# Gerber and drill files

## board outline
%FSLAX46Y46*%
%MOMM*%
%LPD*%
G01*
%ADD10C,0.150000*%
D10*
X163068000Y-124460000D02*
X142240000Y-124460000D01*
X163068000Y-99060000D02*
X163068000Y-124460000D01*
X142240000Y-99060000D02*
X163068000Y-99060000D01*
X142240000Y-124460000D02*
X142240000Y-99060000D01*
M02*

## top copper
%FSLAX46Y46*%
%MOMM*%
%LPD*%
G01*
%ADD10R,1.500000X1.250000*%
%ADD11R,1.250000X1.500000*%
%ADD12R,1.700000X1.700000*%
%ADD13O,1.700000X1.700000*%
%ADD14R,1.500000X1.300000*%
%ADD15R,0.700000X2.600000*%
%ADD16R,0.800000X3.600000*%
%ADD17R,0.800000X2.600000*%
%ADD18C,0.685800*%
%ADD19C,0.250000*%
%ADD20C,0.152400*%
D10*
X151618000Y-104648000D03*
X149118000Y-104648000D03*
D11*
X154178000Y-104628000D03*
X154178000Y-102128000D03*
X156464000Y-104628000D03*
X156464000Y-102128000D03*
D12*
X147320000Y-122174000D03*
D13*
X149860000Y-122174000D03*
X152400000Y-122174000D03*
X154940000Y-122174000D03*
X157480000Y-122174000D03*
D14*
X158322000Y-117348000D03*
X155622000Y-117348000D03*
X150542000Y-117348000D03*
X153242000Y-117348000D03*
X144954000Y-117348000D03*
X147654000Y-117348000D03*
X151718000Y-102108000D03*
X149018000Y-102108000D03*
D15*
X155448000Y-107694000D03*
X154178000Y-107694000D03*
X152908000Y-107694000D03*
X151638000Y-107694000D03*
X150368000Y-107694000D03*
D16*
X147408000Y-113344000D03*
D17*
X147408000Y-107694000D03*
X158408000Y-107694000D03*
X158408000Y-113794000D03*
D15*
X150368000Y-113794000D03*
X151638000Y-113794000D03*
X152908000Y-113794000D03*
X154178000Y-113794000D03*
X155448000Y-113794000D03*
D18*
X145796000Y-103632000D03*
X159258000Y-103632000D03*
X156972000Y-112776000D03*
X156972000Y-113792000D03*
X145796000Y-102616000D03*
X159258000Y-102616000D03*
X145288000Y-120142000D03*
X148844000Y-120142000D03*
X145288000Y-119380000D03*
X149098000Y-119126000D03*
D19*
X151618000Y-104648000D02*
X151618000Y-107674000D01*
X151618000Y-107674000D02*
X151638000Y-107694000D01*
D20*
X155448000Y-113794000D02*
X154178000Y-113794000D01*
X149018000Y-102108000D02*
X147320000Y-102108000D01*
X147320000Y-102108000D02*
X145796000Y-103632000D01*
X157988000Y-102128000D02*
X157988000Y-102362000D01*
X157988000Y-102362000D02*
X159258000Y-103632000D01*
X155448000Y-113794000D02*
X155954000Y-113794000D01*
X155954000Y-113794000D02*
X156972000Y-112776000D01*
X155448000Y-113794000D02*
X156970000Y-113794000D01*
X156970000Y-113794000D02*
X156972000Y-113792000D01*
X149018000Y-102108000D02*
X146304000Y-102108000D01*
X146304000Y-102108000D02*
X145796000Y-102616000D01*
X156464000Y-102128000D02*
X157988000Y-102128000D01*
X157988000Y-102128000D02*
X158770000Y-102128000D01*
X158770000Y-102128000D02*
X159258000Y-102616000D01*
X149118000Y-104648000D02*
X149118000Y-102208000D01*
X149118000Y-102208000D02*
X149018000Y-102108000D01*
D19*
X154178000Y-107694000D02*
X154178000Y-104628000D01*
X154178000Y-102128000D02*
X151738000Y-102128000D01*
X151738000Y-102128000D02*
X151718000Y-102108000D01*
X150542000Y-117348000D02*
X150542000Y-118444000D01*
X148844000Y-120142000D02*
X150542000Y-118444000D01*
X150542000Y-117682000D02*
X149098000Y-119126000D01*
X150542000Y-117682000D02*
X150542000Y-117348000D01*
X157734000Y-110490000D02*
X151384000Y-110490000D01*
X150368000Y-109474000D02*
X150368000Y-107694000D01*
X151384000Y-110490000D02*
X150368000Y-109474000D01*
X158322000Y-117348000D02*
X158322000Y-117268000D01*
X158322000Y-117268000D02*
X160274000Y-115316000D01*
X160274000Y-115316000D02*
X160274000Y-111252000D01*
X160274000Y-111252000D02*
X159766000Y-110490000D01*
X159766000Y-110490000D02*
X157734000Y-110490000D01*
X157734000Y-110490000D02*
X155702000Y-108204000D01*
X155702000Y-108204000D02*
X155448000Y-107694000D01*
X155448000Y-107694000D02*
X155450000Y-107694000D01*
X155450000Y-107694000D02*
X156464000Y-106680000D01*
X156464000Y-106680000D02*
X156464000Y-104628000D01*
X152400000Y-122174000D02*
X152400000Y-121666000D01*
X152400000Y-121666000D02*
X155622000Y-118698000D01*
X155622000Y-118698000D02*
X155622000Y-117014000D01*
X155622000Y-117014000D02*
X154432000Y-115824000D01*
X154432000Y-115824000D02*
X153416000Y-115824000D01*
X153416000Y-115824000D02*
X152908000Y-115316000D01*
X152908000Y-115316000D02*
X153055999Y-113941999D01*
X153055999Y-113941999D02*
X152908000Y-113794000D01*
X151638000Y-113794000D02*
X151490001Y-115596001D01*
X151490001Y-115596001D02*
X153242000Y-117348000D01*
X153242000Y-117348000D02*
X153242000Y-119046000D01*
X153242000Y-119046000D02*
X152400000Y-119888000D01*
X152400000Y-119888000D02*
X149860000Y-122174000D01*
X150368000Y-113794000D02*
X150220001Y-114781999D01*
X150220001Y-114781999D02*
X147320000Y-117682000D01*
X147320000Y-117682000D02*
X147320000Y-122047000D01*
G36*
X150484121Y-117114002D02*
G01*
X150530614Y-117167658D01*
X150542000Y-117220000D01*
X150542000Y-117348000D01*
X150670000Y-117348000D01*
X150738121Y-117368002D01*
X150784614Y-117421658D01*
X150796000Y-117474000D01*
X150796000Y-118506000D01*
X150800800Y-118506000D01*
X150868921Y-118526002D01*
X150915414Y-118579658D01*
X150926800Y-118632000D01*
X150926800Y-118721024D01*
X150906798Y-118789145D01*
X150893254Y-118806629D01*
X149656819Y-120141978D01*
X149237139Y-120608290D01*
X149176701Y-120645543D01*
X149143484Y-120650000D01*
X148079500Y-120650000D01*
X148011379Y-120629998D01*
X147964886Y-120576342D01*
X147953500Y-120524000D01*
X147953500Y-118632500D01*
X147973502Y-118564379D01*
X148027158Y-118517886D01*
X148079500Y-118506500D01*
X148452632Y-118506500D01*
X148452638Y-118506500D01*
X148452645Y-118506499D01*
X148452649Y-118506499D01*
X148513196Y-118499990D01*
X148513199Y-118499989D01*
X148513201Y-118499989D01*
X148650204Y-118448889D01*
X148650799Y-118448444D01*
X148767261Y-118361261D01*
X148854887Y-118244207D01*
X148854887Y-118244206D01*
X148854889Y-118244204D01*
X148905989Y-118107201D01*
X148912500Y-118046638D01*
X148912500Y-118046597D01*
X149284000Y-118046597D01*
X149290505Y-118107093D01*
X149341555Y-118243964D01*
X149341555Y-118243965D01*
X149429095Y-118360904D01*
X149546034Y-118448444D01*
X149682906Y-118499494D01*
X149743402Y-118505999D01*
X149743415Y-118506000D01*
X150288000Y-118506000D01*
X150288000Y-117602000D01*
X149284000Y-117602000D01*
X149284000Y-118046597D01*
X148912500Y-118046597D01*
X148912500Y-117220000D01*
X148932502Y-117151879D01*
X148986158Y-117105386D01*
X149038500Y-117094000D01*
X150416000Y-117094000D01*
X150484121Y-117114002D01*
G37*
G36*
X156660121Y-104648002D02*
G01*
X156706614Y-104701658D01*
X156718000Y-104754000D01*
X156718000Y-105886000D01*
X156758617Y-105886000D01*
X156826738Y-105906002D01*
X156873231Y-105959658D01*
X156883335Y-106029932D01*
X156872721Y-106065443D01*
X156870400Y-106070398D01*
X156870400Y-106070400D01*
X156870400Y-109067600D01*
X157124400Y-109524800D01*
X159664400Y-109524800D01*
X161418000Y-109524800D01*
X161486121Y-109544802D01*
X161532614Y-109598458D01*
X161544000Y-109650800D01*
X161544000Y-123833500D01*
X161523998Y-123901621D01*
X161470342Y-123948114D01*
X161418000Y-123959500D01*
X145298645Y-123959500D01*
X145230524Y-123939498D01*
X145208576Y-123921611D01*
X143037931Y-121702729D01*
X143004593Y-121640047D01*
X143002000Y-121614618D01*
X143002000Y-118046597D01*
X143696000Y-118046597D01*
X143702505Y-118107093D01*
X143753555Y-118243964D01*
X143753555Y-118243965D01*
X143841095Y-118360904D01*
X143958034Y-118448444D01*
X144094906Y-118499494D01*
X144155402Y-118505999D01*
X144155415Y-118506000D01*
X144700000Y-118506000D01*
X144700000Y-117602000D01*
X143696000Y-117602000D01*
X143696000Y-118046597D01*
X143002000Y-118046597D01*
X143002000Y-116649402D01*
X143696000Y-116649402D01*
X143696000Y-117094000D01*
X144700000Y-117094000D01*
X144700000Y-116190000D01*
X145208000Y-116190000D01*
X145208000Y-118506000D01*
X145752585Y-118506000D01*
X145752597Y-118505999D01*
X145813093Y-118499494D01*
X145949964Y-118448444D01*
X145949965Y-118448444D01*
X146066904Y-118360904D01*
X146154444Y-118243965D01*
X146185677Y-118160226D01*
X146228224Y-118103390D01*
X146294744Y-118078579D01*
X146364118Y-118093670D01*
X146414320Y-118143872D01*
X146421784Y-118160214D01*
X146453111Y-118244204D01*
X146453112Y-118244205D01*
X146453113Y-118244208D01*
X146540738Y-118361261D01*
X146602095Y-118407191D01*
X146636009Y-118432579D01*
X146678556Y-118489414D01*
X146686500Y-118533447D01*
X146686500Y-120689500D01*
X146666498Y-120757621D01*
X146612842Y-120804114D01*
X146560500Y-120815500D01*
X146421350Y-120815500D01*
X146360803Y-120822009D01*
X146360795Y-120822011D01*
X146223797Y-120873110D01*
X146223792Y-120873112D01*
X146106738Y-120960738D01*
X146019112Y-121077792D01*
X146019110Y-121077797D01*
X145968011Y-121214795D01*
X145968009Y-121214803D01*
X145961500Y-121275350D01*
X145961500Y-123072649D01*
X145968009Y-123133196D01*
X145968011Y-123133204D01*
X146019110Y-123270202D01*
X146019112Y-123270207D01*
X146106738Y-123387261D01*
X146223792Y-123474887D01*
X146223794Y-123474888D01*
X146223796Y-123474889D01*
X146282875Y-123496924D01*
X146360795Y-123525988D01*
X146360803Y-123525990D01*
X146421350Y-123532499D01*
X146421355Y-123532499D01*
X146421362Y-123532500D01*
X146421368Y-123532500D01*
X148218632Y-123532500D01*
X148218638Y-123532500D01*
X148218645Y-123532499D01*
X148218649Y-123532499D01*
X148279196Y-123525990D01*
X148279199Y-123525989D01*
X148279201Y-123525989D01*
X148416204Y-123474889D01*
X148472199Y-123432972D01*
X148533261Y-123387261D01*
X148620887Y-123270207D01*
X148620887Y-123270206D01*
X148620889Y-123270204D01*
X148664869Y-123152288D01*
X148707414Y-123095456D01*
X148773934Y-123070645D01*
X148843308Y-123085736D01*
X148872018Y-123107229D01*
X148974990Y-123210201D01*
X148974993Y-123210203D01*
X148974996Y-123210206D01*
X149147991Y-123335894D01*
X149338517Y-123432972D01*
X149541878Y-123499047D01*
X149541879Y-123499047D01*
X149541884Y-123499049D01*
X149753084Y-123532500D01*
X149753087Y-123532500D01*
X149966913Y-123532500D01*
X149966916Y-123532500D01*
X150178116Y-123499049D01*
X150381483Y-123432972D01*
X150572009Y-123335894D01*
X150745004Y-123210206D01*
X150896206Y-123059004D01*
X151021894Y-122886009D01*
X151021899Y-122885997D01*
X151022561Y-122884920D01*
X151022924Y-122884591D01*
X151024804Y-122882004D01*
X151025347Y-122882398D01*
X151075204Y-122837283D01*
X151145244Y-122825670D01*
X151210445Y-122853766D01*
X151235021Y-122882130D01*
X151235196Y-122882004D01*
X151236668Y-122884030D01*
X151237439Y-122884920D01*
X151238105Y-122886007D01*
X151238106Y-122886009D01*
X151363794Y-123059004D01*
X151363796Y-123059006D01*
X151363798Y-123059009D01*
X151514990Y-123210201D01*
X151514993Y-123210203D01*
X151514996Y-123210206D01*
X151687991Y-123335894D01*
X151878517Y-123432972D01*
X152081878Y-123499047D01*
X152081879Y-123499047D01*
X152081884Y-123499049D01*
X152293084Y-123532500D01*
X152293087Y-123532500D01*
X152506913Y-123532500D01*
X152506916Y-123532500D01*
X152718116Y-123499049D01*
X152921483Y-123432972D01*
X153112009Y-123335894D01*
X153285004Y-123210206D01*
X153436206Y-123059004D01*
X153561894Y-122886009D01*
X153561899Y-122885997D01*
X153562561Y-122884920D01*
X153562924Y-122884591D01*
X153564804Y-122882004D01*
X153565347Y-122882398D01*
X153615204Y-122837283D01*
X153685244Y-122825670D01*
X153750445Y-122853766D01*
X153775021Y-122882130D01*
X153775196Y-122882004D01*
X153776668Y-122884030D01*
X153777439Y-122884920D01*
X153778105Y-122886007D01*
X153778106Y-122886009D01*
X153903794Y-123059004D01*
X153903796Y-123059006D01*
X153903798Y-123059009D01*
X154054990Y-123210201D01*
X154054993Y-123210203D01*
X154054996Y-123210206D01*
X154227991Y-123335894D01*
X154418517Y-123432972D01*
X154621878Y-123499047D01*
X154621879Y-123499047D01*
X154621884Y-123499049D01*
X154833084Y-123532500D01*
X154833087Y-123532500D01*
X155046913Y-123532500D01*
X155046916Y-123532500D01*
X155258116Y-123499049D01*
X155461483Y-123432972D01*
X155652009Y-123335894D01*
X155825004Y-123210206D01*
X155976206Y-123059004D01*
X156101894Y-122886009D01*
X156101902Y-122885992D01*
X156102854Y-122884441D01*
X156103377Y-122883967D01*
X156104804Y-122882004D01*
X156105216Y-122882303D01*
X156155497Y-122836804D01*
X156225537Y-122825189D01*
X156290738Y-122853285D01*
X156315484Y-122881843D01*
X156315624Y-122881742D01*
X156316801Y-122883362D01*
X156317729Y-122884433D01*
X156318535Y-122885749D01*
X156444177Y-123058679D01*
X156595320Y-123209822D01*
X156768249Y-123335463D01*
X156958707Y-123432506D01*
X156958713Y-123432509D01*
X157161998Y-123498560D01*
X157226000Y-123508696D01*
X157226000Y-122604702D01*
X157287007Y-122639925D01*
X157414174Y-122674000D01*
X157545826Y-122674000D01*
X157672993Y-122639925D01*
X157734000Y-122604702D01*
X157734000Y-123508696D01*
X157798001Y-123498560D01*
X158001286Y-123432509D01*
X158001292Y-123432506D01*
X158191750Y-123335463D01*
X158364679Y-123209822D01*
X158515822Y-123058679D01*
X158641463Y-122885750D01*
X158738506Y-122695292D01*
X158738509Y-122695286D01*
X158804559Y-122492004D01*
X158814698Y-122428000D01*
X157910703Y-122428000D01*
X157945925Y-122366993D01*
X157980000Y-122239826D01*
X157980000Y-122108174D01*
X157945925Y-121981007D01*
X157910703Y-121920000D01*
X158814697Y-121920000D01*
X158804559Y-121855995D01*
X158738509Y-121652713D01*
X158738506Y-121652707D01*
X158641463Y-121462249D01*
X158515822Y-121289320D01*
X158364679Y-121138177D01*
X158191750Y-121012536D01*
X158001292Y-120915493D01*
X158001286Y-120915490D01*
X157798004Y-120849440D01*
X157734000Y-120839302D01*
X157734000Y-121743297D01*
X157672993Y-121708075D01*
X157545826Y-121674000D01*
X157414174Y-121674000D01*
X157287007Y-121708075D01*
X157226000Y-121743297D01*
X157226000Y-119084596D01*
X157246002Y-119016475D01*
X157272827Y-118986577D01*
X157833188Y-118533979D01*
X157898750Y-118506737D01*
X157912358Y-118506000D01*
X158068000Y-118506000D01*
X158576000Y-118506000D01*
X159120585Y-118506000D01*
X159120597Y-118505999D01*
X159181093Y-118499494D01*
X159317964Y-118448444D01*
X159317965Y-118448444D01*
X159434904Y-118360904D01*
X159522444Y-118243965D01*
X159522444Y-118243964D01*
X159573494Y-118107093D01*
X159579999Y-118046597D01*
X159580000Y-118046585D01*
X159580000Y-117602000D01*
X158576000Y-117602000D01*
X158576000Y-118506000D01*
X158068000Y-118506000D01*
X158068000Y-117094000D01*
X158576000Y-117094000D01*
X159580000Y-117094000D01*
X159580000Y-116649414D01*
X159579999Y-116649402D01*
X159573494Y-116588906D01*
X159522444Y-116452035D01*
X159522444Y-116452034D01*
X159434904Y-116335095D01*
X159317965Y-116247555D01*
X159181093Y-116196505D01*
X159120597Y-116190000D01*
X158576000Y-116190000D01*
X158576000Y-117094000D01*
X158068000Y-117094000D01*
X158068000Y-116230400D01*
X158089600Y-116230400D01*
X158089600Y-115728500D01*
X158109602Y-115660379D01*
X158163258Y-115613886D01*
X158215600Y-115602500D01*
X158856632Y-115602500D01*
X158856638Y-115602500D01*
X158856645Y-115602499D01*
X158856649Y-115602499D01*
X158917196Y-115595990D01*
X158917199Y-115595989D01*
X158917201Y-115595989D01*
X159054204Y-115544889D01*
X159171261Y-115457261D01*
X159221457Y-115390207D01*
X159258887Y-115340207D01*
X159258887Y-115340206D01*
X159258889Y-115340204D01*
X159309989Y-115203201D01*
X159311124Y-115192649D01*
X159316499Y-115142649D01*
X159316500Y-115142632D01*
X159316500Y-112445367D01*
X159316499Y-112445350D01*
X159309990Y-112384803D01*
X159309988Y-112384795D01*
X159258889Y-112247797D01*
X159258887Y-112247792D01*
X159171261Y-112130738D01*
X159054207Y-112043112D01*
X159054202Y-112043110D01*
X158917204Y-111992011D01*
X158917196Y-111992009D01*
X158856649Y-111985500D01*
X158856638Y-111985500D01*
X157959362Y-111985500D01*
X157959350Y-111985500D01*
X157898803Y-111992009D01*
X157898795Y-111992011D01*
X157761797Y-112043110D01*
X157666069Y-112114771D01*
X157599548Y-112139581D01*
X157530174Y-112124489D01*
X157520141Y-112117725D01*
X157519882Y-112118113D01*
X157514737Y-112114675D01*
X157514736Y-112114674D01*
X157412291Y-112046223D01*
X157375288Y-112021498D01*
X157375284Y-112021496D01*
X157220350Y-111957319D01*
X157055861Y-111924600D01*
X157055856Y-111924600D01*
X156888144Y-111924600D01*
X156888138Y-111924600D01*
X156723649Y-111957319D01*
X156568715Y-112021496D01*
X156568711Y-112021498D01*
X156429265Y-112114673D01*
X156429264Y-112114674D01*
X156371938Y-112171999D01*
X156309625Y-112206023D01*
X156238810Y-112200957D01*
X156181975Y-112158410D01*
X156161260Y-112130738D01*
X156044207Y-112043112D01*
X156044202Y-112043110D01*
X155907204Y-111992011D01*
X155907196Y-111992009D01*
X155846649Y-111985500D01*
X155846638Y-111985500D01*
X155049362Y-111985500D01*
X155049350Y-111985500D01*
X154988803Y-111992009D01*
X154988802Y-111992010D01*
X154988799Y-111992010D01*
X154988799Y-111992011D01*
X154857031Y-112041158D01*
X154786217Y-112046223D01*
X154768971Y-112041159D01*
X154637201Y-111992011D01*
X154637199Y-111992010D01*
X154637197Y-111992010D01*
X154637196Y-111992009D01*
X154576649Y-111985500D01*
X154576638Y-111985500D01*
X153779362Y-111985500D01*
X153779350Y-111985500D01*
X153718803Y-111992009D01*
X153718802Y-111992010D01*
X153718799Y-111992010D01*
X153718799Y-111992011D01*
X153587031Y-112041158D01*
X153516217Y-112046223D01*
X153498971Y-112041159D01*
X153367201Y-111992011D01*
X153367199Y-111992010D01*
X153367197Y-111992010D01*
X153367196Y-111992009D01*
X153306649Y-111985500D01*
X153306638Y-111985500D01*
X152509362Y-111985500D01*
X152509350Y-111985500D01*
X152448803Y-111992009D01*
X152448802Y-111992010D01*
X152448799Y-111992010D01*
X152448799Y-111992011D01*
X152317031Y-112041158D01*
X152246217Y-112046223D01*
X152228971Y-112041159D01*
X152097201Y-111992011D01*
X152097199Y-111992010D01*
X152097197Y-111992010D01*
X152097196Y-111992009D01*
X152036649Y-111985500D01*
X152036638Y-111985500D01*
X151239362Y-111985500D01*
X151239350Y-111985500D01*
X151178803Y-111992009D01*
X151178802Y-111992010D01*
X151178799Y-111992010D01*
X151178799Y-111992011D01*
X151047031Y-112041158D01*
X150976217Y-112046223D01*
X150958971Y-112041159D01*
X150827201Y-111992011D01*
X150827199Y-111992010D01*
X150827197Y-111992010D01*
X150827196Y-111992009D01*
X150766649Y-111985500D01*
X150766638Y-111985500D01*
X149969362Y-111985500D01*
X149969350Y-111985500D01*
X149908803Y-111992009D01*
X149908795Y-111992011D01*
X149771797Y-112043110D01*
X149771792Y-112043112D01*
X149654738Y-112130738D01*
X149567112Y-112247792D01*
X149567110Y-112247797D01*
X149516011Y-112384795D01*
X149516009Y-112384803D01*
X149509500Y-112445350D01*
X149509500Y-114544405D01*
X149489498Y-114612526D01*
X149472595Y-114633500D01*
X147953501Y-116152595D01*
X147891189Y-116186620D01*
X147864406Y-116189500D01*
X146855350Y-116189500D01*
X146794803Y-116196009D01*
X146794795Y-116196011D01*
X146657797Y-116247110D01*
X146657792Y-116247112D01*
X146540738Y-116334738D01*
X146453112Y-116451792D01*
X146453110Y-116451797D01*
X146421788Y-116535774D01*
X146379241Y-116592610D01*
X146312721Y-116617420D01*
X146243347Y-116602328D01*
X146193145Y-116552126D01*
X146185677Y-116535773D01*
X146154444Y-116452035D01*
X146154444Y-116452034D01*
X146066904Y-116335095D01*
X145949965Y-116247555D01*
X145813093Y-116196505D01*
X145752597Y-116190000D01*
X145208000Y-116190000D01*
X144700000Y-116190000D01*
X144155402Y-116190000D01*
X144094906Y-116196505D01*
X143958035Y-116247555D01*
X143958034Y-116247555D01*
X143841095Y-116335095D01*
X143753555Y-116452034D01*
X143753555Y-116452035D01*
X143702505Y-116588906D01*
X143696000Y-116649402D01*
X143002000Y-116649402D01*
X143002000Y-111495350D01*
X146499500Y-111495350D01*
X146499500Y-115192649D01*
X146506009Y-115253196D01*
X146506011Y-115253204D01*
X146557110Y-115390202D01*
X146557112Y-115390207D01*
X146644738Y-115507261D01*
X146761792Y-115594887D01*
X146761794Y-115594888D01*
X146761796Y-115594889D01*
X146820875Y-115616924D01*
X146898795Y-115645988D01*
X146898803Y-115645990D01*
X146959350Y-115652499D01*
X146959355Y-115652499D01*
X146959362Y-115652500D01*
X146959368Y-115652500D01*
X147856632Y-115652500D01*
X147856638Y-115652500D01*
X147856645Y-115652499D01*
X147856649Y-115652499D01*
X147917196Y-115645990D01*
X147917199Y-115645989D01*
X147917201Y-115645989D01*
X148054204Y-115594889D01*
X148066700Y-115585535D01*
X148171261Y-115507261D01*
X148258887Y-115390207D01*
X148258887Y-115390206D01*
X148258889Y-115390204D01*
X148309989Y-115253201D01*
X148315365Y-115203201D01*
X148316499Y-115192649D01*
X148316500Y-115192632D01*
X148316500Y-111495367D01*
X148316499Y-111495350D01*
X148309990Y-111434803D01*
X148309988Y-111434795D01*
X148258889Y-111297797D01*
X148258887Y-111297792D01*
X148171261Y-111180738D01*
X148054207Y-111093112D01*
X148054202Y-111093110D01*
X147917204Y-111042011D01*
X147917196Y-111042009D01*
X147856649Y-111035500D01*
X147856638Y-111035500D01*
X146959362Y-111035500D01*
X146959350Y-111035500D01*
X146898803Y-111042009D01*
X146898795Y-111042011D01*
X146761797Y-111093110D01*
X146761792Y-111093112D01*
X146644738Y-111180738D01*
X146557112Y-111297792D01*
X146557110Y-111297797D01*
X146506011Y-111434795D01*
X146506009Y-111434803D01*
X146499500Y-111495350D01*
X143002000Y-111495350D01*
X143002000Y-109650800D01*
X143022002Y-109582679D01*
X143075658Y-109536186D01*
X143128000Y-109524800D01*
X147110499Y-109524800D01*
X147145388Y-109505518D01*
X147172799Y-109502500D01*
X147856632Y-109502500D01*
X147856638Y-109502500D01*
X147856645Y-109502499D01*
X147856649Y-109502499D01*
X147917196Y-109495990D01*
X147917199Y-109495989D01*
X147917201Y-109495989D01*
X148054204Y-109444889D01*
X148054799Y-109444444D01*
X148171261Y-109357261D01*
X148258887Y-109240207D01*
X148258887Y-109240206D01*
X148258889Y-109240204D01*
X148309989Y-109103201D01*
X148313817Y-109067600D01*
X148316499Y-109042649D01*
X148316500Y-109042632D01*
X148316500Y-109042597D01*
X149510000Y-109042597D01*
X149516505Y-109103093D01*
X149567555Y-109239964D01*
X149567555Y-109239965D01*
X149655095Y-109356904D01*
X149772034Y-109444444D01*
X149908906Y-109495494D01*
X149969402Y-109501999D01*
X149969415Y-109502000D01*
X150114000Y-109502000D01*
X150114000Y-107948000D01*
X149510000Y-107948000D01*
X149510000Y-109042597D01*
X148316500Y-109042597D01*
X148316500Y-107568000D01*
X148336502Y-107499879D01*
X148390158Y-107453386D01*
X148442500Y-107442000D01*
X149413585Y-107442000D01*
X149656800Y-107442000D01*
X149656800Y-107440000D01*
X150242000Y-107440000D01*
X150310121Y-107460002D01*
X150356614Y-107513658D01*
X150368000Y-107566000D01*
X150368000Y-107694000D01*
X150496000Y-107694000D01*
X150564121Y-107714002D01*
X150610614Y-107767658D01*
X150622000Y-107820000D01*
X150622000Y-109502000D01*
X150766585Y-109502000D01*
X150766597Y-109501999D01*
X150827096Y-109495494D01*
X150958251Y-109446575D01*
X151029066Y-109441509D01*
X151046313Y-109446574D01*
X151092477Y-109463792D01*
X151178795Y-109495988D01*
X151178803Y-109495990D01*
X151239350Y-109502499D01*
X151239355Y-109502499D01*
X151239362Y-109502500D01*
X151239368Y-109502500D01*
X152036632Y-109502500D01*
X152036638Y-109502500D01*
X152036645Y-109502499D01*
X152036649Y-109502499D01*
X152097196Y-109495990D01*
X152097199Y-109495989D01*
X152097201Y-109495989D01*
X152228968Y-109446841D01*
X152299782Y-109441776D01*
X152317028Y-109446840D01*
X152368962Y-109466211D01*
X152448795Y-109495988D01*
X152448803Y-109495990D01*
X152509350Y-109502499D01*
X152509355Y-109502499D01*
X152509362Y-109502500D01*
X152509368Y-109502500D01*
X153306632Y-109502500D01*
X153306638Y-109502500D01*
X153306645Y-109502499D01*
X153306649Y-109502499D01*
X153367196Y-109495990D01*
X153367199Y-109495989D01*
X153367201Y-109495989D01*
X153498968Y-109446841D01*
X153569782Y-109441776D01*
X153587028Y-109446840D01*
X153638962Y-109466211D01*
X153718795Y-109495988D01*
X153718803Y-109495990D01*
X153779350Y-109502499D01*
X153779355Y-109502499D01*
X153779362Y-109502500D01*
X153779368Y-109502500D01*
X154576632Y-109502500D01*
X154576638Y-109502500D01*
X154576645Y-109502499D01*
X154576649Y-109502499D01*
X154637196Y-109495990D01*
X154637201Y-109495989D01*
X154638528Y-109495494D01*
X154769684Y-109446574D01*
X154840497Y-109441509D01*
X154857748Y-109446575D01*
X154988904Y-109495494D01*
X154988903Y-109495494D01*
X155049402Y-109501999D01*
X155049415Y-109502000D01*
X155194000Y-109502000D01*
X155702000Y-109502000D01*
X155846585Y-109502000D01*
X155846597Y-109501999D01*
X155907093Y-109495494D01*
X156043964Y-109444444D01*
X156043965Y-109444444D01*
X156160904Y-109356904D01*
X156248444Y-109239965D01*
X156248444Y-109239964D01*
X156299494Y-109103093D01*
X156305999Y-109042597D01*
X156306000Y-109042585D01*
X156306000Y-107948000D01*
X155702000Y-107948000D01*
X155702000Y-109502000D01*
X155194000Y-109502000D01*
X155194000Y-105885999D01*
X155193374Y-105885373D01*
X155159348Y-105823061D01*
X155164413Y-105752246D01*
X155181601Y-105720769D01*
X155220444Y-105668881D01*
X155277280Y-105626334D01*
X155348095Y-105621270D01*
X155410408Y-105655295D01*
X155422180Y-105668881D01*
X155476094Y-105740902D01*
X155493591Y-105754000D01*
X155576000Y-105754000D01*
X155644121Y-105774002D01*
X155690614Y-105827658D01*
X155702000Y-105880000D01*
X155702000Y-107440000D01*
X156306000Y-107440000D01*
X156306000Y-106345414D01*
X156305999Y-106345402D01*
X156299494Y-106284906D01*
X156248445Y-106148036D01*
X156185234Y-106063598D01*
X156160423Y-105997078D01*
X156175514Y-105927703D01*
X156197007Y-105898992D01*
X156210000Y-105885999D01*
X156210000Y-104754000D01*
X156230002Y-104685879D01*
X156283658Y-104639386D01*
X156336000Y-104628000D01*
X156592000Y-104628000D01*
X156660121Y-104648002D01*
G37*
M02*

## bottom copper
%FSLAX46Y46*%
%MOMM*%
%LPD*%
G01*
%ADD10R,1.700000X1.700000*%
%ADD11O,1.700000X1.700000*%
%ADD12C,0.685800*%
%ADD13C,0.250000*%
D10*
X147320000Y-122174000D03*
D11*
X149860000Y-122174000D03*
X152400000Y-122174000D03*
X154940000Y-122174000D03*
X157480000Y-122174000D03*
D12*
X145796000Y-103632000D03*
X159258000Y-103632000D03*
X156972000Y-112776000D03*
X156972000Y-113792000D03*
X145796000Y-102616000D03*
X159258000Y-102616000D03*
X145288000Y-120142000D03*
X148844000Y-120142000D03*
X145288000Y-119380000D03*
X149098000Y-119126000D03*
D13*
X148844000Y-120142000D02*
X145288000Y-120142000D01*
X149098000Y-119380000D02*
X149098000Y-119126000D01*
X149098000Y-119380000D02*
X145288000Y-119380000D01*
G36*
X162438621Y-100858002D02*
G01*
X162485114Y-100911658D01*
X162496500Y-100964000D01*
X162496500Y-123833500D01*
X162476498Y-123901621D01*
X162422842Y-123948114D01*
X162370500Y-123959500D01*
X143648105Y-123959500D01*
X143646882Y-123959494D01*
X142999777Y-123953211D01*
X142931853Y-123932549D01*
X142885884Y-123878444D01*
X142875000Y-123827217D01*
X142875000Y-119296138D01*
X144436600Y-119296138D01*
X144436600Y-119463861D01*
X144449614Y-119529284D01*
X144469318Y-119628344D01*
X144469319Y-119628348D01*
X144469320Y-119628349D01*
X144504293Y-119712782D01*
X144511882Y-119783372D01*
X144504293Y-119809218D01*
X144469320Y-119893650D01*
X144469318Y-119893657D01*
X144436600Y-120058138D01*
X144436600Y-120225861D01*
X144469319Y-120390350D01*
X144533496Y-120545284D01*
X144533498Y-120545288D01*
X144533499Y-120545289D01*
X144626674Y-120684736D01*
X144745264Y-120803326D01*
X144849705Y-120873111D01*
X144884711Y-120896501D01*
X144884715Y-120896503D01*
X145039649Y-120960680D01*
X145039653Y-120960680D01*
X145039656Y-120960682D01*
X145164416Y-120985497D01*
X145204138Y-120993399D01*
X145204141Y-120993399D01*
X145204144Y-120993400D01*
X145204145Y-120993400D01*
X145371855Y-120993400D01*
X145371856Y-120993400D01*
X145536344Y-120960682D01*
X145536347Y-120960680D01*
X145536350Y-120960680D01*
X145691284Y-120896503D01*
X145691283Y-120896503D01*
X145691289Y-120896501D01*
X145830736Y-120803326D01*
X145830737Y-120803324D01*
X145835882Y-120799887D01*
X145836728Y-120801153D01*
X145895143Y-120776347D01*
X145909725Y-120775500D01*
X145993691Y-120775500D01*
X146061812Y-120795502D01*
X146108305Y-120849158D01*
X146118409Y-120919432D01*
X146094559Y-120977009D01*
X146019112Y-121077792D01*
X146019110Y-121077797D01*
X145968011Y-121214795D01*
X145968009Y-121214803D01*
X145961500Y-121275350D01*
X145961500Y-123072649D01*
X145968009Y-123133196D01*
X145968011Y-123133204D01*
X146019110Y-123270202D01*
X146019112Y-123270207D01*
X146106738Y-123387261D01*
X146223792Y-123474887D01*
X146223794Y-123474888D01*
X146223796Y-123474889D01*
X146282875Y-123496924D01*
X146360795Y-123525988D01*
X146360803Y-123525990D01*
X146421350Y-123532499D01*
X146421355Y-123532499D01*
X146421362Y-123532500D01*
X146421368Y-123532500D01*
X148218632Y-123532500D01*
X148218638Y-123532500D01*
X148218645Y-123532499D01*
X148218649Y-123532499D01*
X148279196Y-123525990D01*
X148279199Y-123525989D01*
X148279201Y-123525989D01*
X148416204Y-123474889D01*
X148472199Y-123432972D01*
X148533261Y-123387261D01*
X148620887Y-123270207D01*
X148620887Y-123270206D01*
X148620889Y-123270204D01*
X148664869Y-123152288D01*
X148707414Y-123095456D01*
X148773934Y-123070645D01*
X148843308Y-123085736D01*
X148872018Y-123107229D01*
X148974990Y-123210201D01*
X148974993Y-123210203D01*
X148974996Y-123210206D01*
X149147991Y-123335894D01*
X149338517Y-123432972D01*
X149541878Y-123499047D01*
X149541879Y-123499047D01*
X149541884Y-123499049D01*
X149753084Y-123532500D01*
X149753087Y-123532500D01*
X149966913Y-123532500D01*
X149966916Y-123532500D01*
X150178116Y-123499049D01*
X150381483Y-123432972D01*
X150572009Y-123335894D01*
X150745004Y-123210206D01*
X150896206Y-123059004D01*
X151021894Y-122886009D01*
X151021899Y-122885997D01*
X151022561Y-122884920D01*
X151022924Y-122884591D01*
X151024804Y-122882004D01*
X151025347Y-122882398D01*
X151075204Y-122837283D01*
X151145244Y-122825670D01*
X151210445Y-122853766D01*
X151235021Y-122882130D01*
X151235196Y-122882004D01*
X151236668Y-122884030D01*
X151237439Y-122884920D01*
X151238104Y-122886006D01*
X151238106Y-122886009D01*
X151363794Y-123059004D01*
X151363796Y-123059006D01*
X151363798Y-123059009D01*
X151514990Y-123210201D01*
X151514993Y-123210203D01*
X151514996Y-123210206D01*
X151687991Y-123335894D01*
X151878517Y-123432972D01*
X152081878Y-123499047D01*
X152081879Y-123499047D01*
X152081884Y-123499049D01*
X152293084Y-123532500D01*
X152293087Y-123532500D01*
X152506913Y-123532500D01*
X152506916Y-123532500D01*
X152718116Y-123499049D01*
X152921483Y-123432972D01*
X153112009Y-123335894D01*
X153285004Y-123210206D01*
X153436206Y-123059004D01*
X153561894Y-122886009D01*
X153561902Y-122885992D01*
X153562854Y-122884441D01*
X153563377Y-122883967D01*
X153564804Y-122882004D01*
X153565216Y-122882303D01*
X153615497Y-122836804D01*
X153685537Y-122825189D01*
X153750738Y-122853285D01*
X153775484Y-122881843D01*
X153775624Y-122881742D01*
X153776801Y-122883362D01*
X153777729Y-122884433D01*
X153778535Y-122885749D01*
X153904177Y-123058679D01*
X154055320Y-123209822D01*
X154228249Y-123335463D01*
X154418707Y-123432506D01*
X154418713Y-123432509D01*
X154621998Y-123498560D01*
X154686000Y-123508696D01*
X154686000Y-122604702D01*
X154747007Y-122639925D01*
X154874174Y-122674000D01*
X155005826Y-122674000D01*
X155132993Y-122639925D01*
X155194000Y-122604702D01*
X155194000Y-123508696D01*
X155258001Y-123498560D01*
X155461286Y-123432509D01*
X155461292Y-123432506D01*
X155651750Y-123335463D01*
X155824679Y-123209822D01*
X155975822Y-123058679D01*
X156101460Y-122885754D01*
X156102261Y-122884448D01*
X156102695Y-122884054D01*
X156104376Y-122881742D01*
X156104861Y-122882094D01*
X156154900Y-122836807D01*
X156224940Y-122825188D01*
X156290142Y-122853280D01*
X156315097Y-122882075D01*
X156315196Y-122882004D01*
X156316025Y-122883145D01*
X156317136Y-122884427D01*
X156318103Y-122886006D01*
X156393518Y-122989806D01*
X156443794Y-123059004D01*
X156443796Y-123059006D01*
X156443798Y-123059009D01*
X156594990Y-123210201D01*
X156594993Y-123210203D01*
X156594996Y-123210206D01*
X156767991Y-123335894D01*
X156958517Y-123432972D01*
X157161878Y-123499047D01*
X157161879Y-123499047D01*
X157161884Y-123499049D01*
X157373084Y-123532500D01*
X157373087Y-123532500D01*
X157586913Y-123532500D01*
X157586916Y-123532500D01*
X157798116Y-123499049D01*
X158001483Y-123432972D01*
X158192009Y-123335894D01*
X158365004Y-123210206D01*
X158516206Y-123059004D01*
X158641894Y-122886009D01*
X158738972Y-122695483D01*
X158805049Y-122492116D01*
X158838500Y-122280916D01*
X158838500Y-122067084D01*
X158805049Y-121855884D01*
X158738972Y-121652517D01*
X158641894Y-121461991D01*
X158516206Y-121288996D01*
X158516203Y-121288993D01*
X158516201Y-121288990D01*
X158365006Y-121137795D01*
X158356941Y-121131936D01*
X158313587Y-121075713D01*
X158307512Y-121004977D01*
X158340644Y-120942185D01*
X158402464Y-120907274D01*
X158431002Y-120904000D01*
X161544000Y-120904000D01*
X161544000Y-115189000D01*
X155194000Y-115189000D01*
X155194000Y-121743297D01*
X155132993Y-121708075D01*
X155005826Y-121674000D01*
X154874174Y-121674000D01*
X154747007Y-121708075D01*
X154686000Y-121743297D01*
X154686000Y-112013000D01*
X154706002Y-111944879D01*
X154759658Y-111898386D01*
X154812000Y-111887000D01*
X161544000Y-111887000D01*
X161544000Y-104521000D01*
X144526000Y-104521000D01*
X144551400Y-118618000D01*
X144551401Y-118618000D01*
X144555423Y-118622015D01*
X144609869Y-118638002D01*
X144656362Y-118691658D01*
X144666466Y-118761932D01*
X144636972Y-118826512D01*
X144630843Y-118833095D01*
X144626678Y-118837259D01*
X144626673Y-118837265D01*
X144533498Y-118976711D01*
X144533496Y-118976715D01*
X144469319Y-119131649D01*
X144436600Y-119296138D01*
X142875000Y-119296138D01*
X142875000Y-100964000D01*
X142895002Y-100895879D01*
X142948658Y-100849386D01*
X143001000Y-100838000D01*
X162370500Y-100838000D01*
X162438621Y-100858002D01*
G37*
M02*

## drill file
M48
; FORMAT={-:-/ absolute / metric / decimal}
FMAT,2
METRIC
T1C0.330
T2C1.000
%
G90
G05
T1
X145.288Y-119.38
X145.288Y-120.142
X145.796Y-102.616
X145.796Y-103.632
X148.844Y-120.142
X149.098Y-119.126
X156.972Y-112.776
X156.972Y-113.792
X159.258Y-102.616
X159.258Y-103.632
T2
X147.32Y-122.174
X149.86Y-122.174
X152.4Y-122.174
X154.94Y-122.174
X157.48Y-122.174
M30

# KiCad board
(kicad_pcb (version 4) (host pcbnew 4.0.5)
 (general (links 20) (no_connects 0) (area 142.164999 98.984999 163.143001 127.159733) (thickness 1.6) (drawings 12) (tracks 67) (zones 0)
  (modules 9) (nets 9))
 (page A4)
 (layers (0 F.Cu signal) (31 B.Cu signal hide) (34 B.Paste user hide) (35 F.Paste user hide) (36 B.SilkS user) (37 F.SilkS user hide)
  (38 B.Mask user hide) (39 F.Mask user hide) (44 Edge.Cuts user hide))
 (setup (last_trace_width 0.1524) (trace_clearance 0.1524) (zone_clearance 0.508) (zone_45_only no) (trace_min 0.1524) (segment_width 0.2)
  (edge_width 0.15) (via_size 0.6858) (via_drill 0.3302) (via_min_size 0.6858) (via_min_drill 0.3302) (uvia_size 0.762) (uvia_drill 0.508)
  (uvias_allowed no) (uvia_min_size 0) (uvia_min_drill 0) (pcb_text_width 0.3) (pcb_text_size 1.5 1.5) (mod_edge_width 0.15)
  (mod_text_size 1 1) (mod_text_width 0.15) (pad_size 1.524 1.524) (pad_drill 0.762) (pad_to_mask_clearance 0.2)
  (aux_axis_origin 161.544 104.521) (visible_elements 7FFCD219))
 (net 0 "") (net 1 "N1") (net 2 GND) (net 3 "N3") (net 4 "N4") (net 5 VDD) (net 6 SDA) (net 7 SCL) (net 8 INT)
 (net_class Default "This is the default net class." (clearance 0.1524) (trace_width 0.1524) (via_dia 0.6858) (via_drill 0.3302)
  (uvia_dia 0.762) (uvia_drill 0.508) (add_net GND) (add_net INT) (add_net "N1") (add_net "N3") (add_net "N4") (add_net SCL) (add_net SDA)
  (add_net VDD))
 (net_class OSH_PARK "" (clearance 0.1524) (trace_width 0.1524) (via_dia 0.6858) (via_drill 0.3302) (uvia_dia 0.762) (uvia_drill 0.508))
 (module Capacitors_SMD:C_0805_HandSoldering (layer F.Cu) (at 150.368 104.648 180)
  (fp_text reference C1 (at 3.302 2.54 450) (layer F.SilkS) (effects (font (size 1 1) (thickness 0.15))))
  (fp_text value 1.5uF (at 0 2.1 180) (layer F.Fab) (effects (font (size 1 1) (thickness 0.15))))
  (pad 1 smd rect (at -1.25 0 180) (size 1.5 1.25) (layers F.Cu F.Paste F.Mask) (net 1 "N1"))
  (pad 2 smd rect (at 1.25 0 180) (size 1.5 1.25) (layers F.Cu F.Paste F.Mask) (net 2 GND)))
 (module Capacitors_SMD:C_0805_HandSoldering (layer F.Cu) (at 154.178 103.378 90)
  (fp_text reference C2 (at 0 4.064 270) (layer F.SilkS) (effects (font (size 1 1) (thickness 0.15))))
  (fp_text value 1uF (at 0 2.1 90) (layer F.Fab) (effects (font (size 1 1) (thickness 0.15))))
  (pad 1 smd rect (at -1.25 0 90) (size 1.5 1.25) (layers F.Cu F.Paste F.Mask) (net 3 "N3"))
  (pad 2 smd rect (at 1.25 0 90) (size 1.5 1.25) (layers F.Cu F.Paste F.Mask) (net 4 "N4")))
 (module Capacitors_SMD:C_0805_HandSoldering (layer F.Cu) (at 156.464 103.378 90)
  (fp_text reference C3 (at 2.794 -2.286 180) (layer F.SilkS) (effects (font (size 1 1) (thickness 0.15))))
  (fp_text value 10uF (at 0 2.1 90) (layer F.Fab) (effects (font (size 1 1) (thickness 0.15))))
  (pad 1 smd rect (at -1.25 0 90) (size 1.5 1.25) (layers F.Cu F.Paste F.Mask) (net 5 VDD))
  (pad 2 smd rect (at 1.25 0 90) (size 1.5 1.25) (layers F.Cu F.Paste F.Mask) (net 2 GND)))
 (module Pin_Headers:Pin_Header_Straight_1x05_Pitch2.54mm (layer F.Cu) (at 147.32 122.174 90)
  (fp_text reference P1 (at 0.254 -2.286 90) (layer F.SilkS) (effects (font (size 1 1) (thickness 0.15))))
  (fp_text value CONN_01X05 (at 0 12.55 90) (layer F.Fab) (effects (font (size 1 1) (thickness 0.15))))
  (pad 1 thru_hole rect (at 0 0 90) (size 1.7 1.7) (drill 1) (layers *.Cu *.Mask) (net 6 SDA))
  (pad 2 thru_hole oval (at 0 2.54 90) (size 1.7 1.7) (drill 1) (layers *.Cu *.Mask) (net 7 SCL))
  (pad 3 thru_hole oval (at 0 5.08 90) (size 1.7 1.7) (drill 1) (layers *.Cu *.Mask) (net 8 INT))
  (pad 4 thru_hole oval (at 0 7.62 90) (size 1.7 1.7) (drill 1) (layers *.Cu *.Mask) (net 2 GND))
  (pad 5 thru_hole oval (at 0 10.16 90) (size 1.7 1.7) (drill 1) (layers *.Cu *.Mask) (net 5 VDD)))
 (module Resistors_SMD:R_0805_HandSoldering (layer F.Cu) (at 156.972 117.348 180)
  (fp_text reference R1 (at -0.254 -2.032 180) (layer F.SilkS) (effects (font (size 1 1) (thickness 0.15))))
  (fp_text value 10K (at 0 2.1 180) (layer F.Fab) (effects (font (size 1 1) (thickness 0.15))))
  (pad 1 smd rect (at -1.35 0 180) (size 1.5 1.3) (layers F.Cu F.Paste F.Mask) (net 5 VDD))
  (pad 2 smd rect (at 1.35 0 180) (size 1.5 1.3) (layers F.Cu F.Paste F.Mask) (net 8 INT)))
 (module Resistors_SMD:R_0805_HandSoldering (layer F.Cu) (at 151.892 117.348)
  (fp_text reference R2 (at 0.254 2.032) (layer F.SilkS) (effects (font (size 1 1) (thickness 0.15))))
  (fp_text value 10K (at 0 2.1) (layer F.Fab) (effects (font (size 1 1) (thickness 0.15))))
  (pad 1 smd rect (at -1.35 0) (size 1.5 1.3) (layers F.Cu F.Paste F.Mask) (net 5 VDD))
  (pad 2 smd rect (at 1.35 0) (size 1.5 1.3) (layers F.Cu F.Paste F.Mask) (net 7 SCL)))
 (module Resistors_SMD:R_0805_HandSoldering (layer F.Cu) (at 146.304 117.348)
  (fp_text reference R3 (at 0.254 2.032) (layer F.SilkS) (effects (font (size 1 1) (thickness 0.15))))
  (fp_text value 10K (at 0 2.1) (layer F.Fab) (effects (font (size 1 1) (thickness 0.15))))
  (pad 1 smd rect (at -1.35 0) (size 1.5 1.3) (layers F.Cu F.Paste F.Mask) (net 5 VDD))
  (pad 2 smd rect (at 1.35 0) (size 1.5 1.3) (layers F.Cu F.Paste F.Mask) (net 6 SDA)))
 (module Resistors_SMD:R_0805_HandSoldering (layer F.Cu) (at 150.368 102.108 180)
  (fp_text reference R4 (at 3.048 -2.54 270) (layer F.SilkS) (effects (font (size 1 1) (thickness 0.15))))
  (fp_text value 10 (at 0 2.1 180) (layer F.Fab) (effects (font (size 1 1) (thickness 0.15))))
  (pad 1 smd rect (at -1.35 0 180) (size 1.5 1.3) (layers F.Cu F.Paste F.Mask) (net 4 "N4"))
  (pad 2 smd rect (at 1.35 0 180) (size 1.5 1.3) (layers F.Cu F.Paste F.Mask) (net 2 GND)))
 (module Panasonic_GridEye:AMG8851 (layer F.Cu) (at 152.908 110.744)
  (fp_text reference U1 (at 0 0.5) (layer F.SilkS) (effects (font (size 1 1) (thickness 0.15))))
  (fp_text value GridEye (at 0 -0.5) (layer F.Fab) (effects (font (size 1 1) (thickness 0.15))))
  (pad 9 smd rect (at 2.54 -3.05) (size 0.7 2.6) (layers F.Cu F.Paste F.Mask) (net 5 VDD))
  (pad 10 smd rect (at 1.27 -3.05) (size 0.7 2.6) (layers F.Cu F.Paste F.Mask) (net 3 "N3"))
  (pad 11 smd rect (at 0 -3.05) (size 0.7 2.6) (layers F.Cu F.Paste F.Mask))
  (pad 12 smd rect (at -1.27 -3.05) (size 0.7 2.6) (layers F.Cu F.Paste F.Mask) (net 1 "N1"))
  (pad 13 smd rect (at -2.54 -3.05) (size 0.7 2.6) (layers F.Cu F.Paste F.Mask) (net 5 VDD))
  (pad 1 smd rect (at -5.5 2.6) (size 0.8 3.6) (layers F.Cu F.Paste F.Mask))
  (pad 14 smd rect (at -5.5 -3.05) (size 0.8 2.6) (layers F.Cu F.Paste F.Mask))
  (pad 8 smd rect (at 5.5 -3.05) (size 0.8 2.6) (layers F.Cu F.Paste F.Mask))
  (pad 7 smd rect (at 5.5 3.05) (size 0.8 2.6) (layers F.Cu F.Paste F.Mask))
  (pad 2 smd rect (at -2.54 3.05) (size 0.7 2.6) (layers F.Cu F.Paste F.Mask) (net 6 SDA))
  (pad 3 smd rect (at -1.27 3.05) (size 0.7 2.6) (layers F.Cu F.Paste F.Mask) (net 7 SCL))
  (pad 4 smd rect (at 0 3.05) (size 0.7 2.6) (layers F.Cu F.Paste F.Mask) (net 8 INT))
  (pad 5 smd rect (at 1.27 3.05) (size 0.7 2.6) (layers F.Cu F.Paste F.Mask) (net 2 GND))
  (pad 6 smd rect (at 2.54 3.05) (size 0.7 2.6) (layers F.Cu F.Paste F.Mask) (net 2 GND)))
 (gr_line (start 163.068 124.46) (end 142.24 124.46) (angle 90) (layer Edge.Cuts) (width 0.15))
 (gr_line (start 163.068 99.06) (end 163.068 124.46) (angle 90) (layer Edge.Cuts) (width 0.15))
 (gr_line (start 142.24 99.06) (end 163.068 99.06) (angle 90) (layer Edge.Cuts) (width 0.15))
 (gr_line (start 142.24 124.46) (end 142.24 99.06) (angle 90) (layer Edge.Cuts) (width 0.15))
 (segment (start 151.618 104.648) (end 151.618 107.674) (width 0.25) (layer F.Cu) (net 1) (status 20))
 (segment (start 151.618 107.674) (end 151.638 107.694) (width 0.25) (layer F.Cu) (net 1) (status 30))
 (segment (start 155.448 113.794) (end 154.178 113.794) (width 0.1524) (layer F.Cu) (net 2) (status 30))
 (via (at 145.796 103.632) (size 0.6858) (drill 0.3302) (layers F.Cu B.Cu) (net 2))
 (segment (start 149.018 102.108) (end 147.32 102.108) (width 0.1524) (layer F.Cu) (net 2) (status 10))
 (segment (start 147.32 102.108) (end 145.796 103.632) (width 0.1524) (layer F.Cu) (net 2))
 (via (at 159.258 103.632) (size 0.6858) (drill 0.3302) (layers F.Cu B.Cu) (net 2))
 (segment (start 157.988 102.128) (end 157.988 102.362) (width 0.1524) (layer F.Cu) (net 2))
 (segment (start 157.988 102.362) (end 159.258 103.632) (width 0.1524) (layer F.Cu) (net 2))
 (via (at 156.972 112.776) (size 0.6858) (drill 0.3302) (layers F.Cu B.Cu) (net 2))
 (segment (start 155.448 113.794) (end 155.954 113.794) (width 0.1524) (layer F.Cu) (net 2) (status 10))
 (segment (start 155.954 113.794) (end 156.972 112.776) (width 0.1524) (layer F.Cu) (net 2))
 (via (at 156.972 113.792) (size 0.6858) (drill 0.3302) (layers F.Cu B.Cu) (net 2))
 (segment (start 155.448 113.794) (end 156.97 113.794) (width 0.1524) (layer F.Cu) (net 2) (status 10))
 (segment (start 156.97 113.794) (end 156.972 113.792) (width 0.1524) (layer F.Cu) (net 2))
 (via (at 145.796 102.616) (size 0.6858) (drill 0.3302) (layers F.Cu B.Cu) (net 2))
 (segment (start 149.018 102.108) (end 146.304 102.108) (width 0.1524) (layer F.Cu) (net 2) (status 10))
 (segment (start 146.304 102.108) (end 145.796 102.616) (width 0.1524) (layer F.Cu) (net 2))
 (via (at 159.258 102.616) (size 0.6858) (drill 0.3302) (layers F.Cu B.Cu) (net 2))
 (segment (start 156.464 102.128) (end 157.988 102.128) (width 0.1524) (layer F.Cu) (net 2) (status 10))
 (segment (start 157.988 102.128) (end 158.77 102.128) (width 0.1524) (layer F.Cu) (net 2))
 (segment (start 158.77 102.128) (end 159.258 102.616) (width 0.1524) (layer F.Cu) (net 2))
 (segment (start 149.118 104.648) (end 149.118 102.208) (width 0.1524) (layer F.Cu) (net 2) (status 30))
 (segment (start 149.118 102.208) (end 149.018 102.108) (width 0.1524) (layer F.Cu) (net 2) (status 30))
 (segment (start 154.178 107.694) (end 154.178 104.628) (width 0.25) (layer F.Cu) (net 3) (status 10))
 (segment (start 154.178 102.128) (end 151.738 102.128) (width 0.25) (layer F.Cu) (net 4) (status 30))
 (segment (start 151.738 102.128) (end 151.718 102.108) (width 0.25) (layer F.Cu) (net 4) (status 30))
 (via (at 145.288 120.142) (size 0.6858) (drill 0.3302) (layers F.Cu B.Cu) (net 5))
 (segment (start 150.542 117.348) (end 150.542 118.444) (width 0.25) (layer F.Cu) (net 5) (status 10))
 (segment (start 148.844 120.142) (end 150.542 118.444) (width 0.25) (layer F.Cu) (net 5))
 (via (at 148.844 120.142) (size 0.6858) (drill 0.3302) (layers F.Cu B.Cu) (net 5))
 (segment (start 148.844 120.142) (end 145.288 120.142) (width 0.25) (layer B.Cu) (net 5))
 (via (at 145.288 119.38) (size 0.6858) (drill 0.3302) (layers F.Cu B.Cu) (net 5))
 (segment (start 150.542 117.682) (end 149.098 119.126) (width 0.25) (layer F.Cu) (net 5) (status 10))
 (via (at 149.098 119.126) (size 0.6858) (drill 0.3302) (layers F.Cu B.Cu) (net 5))
 (segment (start 149.098 119.38) (end 149.098 119.126) (width 0.25) (layer B.Cu) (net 5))
 (segment (start 149.098 119.38) (end 145.288 119.38) (width 0.25) (layer B.Cu) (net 5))
 (segment (start 150.542 117.682) (end 150.542 117.348) (width 0.25) (layer F.Cu) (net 5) (status 30))
 (segment (start 157.734 110.49) (end 151.384 110.49) (width 0.25) (layer F.Cu) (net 5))
 (segment (start 150.368 109.474) (end 150.368 107.694) (width 0.25) (layer F.Cu) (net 5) (status 20))
 (segment (start 151.384 110.49) (end 150.368 109.474) (width 0.25) (layer F.Cu) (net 5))
 (segment (start 158.322 117.348) (end 158.322 117.268) (width 0.25) (layer F.Cu) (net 5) (status 30))
 (segment (start 158.322 117.268) (end 160.274 115.316) (width 0.25) (layer F.Cu) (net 5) (status 10))
 (segment (start 160.274 115.316) (end 160.274 111.252) (width 0.25) (layer F.Cu) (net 5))
 (segment (start 160.274 111.252) (end 159.766 110.49) (width 0.25) (layer F.Cu) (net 5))
 (segment (start 159.766 110.49) (end 157.734 110.49) (width 0.25) (layer F.Cu) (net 5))
 (segment (start 157.734 110.49) (end 155.702 108.204) (width 0.25) (layer F.Cu) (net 5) (status 20))
 (segment (start 155.702 108.204) (end 155.448 107.694) (width 0.25) (layer F.Cu) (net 5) (status 30))
 (segment (start 155.448 107.694) (end 155.45 107.694) (width 0.25) (layer F.Cu) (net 5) (status 30))
 (segment (start 155.45 107.694) (end 156.464 106.68) (width 0.25) (layer F.Cu) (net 5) (status 10))
 (segment (start 156.464 106.68) (end 156.464 104.628) (width 0.25) (layer F.Cu) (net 5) (status 20))
 (segment (start 152.4 122.174) (end 152.4 121.666) (width 0.25) (layer F.Cu) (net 8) (status 30))
 (segment (start 152.4 121.666) (end 155.622 118.698) (width 0.25) (layer F.Cu) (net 8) (status 10))
 (segment (start 155.622 118.698) (end 155.622 117.014) (width 0.25) (layer F.Cu) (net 8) (status 20))
 (segment (start 155.622 117.014) (end 154.432 115.824) (width 0.25) (layer F.Cu) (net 8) (status 10))
 (segment (start 154.432 115.824) (end 153.416 115.824) (width 0.25) (layer F.Cu) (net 8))
 (segment (start 153.416 115.824) (end 152.908 115.316) (width 0.25) (layer F.Cu) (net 8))
 (segment (start 152.908 115.316) (end 153.055999 113.941999) (width 0.25) (layer F.Cu) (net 8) (status 20))
 (segment (start 153.055999 113.941999) (end 152.908 113.794) (width 0.25) (layer F.Cu) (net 8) (status 30))
 (segment (start 151.638 113.794) (end 151.490001 115.596001) (width 0.25) (layer F.Cu) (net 7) (status 10))
 (segment (start 151.490001 115.596001) (end 153.242 117.348) (width 0.25) (layer F.Cu) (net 7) (status 20))
 (segment (start 153.242 117.348) (end 153.242 119.046) (width 0.25) (layer F.Cu) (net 7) (status 10))
 (segment (start 153.242 119.046) (end 152.4 119.888) (width 0.25) (layer F.Cu) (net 7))
 (segment (start 152.4 119.888) (end 149.86 122.174) (width 0.25) (layer F.Cu) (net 7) (status 20))
 (segment (start 150.368 113.794) (end 150.220001 114.781999) (width 0.25) (layer F.Cu) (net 6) (status 30))
 (segment (start 150.220001 114.781999) (end 147.32 117.682) (width 0.25) (layer F.Cu) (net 6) (status 10))
 (segment (start 147.32 117.682) (end 147.32 122.047) (width 0.25) (layer F.Cu) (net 6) (status 30))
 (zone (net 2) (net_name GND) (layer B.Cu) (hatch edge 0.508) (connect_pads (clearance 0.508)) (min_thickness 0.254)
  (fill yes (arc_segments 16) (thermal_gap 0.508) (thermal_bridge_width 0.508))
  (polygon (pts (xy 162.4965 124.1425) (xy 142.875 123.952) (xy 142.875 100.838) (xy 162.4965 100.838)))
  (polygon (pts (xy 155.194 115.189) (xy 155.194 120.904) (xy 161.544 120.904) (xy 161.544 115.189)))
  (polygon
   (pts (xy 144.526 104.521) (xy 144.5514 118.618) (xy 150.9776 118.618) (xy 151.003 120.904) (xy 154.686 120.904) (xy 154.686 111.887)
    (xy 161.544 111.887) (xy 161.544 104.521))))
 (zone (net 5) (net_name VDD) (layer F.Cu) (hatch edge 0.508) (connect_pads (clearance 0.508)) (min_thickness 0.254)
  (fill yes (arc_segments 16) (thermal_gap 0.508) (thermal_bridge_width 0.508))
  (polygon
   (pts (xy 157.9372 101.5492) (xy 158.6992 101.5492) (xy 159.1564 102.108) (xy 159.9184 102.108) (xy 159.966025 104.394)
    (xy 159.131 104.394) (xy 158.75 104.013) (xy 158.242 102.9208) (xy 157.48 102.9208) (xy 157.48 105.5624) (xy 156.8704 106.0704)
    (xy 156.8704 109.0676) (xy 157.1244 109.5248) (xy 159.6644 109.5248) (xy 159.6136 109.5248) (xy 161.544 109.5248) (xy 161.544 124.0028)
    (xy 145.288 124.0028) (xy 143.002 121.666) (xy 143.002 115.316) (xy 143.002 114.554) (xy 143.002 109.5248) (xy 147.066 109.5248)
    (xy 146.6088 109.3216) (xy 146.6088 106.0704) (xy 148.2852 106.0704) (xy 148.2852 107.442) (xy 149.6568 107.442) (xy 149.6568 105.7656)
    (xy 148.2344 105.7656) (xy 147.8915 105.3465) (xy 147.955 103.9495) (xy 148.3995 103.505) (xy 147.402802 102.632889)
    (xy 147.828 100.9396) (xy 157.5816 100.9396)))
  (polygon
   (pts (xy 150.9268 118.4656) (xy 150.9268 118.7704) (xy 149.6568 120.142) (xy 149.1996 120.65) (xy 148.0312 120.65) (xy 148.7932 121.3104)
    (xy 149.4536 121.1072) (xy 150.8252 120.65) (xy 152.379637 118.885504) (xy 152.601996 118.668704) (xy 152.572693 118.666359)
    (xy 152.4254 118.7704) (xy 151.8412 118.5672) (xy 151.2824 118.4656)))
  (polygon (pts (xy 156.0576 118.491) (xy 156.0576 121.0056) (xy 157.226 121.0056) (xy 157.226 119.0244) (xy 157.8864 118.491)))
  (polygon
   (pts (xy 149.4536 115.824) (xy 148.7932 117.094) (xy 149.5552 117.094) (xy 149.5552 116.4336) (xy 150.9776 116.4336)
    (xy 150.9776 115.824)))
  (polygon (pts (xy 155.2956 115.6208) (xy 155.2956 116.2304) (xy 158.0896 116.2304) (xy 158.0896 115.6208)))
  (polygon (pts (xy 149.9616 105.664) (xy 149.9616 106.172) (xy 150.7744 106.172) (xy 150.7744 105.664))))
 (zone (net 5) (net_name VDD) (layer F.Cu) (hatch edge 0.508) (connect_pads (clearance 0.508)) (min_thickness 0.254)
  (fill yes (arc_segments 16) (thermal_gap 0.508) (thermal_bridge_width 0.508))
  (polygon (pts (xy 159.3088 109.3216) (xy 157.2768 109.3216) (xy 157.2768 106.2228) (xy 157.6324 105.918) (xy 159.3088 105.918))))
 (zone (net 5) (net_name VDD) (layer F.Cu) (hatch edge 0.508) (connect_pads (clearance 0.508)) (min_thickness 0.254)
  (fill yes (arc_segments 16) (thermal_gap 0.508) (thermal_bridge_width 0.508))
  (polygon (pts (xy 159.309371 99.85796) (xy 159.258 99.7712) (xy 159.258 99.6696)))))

